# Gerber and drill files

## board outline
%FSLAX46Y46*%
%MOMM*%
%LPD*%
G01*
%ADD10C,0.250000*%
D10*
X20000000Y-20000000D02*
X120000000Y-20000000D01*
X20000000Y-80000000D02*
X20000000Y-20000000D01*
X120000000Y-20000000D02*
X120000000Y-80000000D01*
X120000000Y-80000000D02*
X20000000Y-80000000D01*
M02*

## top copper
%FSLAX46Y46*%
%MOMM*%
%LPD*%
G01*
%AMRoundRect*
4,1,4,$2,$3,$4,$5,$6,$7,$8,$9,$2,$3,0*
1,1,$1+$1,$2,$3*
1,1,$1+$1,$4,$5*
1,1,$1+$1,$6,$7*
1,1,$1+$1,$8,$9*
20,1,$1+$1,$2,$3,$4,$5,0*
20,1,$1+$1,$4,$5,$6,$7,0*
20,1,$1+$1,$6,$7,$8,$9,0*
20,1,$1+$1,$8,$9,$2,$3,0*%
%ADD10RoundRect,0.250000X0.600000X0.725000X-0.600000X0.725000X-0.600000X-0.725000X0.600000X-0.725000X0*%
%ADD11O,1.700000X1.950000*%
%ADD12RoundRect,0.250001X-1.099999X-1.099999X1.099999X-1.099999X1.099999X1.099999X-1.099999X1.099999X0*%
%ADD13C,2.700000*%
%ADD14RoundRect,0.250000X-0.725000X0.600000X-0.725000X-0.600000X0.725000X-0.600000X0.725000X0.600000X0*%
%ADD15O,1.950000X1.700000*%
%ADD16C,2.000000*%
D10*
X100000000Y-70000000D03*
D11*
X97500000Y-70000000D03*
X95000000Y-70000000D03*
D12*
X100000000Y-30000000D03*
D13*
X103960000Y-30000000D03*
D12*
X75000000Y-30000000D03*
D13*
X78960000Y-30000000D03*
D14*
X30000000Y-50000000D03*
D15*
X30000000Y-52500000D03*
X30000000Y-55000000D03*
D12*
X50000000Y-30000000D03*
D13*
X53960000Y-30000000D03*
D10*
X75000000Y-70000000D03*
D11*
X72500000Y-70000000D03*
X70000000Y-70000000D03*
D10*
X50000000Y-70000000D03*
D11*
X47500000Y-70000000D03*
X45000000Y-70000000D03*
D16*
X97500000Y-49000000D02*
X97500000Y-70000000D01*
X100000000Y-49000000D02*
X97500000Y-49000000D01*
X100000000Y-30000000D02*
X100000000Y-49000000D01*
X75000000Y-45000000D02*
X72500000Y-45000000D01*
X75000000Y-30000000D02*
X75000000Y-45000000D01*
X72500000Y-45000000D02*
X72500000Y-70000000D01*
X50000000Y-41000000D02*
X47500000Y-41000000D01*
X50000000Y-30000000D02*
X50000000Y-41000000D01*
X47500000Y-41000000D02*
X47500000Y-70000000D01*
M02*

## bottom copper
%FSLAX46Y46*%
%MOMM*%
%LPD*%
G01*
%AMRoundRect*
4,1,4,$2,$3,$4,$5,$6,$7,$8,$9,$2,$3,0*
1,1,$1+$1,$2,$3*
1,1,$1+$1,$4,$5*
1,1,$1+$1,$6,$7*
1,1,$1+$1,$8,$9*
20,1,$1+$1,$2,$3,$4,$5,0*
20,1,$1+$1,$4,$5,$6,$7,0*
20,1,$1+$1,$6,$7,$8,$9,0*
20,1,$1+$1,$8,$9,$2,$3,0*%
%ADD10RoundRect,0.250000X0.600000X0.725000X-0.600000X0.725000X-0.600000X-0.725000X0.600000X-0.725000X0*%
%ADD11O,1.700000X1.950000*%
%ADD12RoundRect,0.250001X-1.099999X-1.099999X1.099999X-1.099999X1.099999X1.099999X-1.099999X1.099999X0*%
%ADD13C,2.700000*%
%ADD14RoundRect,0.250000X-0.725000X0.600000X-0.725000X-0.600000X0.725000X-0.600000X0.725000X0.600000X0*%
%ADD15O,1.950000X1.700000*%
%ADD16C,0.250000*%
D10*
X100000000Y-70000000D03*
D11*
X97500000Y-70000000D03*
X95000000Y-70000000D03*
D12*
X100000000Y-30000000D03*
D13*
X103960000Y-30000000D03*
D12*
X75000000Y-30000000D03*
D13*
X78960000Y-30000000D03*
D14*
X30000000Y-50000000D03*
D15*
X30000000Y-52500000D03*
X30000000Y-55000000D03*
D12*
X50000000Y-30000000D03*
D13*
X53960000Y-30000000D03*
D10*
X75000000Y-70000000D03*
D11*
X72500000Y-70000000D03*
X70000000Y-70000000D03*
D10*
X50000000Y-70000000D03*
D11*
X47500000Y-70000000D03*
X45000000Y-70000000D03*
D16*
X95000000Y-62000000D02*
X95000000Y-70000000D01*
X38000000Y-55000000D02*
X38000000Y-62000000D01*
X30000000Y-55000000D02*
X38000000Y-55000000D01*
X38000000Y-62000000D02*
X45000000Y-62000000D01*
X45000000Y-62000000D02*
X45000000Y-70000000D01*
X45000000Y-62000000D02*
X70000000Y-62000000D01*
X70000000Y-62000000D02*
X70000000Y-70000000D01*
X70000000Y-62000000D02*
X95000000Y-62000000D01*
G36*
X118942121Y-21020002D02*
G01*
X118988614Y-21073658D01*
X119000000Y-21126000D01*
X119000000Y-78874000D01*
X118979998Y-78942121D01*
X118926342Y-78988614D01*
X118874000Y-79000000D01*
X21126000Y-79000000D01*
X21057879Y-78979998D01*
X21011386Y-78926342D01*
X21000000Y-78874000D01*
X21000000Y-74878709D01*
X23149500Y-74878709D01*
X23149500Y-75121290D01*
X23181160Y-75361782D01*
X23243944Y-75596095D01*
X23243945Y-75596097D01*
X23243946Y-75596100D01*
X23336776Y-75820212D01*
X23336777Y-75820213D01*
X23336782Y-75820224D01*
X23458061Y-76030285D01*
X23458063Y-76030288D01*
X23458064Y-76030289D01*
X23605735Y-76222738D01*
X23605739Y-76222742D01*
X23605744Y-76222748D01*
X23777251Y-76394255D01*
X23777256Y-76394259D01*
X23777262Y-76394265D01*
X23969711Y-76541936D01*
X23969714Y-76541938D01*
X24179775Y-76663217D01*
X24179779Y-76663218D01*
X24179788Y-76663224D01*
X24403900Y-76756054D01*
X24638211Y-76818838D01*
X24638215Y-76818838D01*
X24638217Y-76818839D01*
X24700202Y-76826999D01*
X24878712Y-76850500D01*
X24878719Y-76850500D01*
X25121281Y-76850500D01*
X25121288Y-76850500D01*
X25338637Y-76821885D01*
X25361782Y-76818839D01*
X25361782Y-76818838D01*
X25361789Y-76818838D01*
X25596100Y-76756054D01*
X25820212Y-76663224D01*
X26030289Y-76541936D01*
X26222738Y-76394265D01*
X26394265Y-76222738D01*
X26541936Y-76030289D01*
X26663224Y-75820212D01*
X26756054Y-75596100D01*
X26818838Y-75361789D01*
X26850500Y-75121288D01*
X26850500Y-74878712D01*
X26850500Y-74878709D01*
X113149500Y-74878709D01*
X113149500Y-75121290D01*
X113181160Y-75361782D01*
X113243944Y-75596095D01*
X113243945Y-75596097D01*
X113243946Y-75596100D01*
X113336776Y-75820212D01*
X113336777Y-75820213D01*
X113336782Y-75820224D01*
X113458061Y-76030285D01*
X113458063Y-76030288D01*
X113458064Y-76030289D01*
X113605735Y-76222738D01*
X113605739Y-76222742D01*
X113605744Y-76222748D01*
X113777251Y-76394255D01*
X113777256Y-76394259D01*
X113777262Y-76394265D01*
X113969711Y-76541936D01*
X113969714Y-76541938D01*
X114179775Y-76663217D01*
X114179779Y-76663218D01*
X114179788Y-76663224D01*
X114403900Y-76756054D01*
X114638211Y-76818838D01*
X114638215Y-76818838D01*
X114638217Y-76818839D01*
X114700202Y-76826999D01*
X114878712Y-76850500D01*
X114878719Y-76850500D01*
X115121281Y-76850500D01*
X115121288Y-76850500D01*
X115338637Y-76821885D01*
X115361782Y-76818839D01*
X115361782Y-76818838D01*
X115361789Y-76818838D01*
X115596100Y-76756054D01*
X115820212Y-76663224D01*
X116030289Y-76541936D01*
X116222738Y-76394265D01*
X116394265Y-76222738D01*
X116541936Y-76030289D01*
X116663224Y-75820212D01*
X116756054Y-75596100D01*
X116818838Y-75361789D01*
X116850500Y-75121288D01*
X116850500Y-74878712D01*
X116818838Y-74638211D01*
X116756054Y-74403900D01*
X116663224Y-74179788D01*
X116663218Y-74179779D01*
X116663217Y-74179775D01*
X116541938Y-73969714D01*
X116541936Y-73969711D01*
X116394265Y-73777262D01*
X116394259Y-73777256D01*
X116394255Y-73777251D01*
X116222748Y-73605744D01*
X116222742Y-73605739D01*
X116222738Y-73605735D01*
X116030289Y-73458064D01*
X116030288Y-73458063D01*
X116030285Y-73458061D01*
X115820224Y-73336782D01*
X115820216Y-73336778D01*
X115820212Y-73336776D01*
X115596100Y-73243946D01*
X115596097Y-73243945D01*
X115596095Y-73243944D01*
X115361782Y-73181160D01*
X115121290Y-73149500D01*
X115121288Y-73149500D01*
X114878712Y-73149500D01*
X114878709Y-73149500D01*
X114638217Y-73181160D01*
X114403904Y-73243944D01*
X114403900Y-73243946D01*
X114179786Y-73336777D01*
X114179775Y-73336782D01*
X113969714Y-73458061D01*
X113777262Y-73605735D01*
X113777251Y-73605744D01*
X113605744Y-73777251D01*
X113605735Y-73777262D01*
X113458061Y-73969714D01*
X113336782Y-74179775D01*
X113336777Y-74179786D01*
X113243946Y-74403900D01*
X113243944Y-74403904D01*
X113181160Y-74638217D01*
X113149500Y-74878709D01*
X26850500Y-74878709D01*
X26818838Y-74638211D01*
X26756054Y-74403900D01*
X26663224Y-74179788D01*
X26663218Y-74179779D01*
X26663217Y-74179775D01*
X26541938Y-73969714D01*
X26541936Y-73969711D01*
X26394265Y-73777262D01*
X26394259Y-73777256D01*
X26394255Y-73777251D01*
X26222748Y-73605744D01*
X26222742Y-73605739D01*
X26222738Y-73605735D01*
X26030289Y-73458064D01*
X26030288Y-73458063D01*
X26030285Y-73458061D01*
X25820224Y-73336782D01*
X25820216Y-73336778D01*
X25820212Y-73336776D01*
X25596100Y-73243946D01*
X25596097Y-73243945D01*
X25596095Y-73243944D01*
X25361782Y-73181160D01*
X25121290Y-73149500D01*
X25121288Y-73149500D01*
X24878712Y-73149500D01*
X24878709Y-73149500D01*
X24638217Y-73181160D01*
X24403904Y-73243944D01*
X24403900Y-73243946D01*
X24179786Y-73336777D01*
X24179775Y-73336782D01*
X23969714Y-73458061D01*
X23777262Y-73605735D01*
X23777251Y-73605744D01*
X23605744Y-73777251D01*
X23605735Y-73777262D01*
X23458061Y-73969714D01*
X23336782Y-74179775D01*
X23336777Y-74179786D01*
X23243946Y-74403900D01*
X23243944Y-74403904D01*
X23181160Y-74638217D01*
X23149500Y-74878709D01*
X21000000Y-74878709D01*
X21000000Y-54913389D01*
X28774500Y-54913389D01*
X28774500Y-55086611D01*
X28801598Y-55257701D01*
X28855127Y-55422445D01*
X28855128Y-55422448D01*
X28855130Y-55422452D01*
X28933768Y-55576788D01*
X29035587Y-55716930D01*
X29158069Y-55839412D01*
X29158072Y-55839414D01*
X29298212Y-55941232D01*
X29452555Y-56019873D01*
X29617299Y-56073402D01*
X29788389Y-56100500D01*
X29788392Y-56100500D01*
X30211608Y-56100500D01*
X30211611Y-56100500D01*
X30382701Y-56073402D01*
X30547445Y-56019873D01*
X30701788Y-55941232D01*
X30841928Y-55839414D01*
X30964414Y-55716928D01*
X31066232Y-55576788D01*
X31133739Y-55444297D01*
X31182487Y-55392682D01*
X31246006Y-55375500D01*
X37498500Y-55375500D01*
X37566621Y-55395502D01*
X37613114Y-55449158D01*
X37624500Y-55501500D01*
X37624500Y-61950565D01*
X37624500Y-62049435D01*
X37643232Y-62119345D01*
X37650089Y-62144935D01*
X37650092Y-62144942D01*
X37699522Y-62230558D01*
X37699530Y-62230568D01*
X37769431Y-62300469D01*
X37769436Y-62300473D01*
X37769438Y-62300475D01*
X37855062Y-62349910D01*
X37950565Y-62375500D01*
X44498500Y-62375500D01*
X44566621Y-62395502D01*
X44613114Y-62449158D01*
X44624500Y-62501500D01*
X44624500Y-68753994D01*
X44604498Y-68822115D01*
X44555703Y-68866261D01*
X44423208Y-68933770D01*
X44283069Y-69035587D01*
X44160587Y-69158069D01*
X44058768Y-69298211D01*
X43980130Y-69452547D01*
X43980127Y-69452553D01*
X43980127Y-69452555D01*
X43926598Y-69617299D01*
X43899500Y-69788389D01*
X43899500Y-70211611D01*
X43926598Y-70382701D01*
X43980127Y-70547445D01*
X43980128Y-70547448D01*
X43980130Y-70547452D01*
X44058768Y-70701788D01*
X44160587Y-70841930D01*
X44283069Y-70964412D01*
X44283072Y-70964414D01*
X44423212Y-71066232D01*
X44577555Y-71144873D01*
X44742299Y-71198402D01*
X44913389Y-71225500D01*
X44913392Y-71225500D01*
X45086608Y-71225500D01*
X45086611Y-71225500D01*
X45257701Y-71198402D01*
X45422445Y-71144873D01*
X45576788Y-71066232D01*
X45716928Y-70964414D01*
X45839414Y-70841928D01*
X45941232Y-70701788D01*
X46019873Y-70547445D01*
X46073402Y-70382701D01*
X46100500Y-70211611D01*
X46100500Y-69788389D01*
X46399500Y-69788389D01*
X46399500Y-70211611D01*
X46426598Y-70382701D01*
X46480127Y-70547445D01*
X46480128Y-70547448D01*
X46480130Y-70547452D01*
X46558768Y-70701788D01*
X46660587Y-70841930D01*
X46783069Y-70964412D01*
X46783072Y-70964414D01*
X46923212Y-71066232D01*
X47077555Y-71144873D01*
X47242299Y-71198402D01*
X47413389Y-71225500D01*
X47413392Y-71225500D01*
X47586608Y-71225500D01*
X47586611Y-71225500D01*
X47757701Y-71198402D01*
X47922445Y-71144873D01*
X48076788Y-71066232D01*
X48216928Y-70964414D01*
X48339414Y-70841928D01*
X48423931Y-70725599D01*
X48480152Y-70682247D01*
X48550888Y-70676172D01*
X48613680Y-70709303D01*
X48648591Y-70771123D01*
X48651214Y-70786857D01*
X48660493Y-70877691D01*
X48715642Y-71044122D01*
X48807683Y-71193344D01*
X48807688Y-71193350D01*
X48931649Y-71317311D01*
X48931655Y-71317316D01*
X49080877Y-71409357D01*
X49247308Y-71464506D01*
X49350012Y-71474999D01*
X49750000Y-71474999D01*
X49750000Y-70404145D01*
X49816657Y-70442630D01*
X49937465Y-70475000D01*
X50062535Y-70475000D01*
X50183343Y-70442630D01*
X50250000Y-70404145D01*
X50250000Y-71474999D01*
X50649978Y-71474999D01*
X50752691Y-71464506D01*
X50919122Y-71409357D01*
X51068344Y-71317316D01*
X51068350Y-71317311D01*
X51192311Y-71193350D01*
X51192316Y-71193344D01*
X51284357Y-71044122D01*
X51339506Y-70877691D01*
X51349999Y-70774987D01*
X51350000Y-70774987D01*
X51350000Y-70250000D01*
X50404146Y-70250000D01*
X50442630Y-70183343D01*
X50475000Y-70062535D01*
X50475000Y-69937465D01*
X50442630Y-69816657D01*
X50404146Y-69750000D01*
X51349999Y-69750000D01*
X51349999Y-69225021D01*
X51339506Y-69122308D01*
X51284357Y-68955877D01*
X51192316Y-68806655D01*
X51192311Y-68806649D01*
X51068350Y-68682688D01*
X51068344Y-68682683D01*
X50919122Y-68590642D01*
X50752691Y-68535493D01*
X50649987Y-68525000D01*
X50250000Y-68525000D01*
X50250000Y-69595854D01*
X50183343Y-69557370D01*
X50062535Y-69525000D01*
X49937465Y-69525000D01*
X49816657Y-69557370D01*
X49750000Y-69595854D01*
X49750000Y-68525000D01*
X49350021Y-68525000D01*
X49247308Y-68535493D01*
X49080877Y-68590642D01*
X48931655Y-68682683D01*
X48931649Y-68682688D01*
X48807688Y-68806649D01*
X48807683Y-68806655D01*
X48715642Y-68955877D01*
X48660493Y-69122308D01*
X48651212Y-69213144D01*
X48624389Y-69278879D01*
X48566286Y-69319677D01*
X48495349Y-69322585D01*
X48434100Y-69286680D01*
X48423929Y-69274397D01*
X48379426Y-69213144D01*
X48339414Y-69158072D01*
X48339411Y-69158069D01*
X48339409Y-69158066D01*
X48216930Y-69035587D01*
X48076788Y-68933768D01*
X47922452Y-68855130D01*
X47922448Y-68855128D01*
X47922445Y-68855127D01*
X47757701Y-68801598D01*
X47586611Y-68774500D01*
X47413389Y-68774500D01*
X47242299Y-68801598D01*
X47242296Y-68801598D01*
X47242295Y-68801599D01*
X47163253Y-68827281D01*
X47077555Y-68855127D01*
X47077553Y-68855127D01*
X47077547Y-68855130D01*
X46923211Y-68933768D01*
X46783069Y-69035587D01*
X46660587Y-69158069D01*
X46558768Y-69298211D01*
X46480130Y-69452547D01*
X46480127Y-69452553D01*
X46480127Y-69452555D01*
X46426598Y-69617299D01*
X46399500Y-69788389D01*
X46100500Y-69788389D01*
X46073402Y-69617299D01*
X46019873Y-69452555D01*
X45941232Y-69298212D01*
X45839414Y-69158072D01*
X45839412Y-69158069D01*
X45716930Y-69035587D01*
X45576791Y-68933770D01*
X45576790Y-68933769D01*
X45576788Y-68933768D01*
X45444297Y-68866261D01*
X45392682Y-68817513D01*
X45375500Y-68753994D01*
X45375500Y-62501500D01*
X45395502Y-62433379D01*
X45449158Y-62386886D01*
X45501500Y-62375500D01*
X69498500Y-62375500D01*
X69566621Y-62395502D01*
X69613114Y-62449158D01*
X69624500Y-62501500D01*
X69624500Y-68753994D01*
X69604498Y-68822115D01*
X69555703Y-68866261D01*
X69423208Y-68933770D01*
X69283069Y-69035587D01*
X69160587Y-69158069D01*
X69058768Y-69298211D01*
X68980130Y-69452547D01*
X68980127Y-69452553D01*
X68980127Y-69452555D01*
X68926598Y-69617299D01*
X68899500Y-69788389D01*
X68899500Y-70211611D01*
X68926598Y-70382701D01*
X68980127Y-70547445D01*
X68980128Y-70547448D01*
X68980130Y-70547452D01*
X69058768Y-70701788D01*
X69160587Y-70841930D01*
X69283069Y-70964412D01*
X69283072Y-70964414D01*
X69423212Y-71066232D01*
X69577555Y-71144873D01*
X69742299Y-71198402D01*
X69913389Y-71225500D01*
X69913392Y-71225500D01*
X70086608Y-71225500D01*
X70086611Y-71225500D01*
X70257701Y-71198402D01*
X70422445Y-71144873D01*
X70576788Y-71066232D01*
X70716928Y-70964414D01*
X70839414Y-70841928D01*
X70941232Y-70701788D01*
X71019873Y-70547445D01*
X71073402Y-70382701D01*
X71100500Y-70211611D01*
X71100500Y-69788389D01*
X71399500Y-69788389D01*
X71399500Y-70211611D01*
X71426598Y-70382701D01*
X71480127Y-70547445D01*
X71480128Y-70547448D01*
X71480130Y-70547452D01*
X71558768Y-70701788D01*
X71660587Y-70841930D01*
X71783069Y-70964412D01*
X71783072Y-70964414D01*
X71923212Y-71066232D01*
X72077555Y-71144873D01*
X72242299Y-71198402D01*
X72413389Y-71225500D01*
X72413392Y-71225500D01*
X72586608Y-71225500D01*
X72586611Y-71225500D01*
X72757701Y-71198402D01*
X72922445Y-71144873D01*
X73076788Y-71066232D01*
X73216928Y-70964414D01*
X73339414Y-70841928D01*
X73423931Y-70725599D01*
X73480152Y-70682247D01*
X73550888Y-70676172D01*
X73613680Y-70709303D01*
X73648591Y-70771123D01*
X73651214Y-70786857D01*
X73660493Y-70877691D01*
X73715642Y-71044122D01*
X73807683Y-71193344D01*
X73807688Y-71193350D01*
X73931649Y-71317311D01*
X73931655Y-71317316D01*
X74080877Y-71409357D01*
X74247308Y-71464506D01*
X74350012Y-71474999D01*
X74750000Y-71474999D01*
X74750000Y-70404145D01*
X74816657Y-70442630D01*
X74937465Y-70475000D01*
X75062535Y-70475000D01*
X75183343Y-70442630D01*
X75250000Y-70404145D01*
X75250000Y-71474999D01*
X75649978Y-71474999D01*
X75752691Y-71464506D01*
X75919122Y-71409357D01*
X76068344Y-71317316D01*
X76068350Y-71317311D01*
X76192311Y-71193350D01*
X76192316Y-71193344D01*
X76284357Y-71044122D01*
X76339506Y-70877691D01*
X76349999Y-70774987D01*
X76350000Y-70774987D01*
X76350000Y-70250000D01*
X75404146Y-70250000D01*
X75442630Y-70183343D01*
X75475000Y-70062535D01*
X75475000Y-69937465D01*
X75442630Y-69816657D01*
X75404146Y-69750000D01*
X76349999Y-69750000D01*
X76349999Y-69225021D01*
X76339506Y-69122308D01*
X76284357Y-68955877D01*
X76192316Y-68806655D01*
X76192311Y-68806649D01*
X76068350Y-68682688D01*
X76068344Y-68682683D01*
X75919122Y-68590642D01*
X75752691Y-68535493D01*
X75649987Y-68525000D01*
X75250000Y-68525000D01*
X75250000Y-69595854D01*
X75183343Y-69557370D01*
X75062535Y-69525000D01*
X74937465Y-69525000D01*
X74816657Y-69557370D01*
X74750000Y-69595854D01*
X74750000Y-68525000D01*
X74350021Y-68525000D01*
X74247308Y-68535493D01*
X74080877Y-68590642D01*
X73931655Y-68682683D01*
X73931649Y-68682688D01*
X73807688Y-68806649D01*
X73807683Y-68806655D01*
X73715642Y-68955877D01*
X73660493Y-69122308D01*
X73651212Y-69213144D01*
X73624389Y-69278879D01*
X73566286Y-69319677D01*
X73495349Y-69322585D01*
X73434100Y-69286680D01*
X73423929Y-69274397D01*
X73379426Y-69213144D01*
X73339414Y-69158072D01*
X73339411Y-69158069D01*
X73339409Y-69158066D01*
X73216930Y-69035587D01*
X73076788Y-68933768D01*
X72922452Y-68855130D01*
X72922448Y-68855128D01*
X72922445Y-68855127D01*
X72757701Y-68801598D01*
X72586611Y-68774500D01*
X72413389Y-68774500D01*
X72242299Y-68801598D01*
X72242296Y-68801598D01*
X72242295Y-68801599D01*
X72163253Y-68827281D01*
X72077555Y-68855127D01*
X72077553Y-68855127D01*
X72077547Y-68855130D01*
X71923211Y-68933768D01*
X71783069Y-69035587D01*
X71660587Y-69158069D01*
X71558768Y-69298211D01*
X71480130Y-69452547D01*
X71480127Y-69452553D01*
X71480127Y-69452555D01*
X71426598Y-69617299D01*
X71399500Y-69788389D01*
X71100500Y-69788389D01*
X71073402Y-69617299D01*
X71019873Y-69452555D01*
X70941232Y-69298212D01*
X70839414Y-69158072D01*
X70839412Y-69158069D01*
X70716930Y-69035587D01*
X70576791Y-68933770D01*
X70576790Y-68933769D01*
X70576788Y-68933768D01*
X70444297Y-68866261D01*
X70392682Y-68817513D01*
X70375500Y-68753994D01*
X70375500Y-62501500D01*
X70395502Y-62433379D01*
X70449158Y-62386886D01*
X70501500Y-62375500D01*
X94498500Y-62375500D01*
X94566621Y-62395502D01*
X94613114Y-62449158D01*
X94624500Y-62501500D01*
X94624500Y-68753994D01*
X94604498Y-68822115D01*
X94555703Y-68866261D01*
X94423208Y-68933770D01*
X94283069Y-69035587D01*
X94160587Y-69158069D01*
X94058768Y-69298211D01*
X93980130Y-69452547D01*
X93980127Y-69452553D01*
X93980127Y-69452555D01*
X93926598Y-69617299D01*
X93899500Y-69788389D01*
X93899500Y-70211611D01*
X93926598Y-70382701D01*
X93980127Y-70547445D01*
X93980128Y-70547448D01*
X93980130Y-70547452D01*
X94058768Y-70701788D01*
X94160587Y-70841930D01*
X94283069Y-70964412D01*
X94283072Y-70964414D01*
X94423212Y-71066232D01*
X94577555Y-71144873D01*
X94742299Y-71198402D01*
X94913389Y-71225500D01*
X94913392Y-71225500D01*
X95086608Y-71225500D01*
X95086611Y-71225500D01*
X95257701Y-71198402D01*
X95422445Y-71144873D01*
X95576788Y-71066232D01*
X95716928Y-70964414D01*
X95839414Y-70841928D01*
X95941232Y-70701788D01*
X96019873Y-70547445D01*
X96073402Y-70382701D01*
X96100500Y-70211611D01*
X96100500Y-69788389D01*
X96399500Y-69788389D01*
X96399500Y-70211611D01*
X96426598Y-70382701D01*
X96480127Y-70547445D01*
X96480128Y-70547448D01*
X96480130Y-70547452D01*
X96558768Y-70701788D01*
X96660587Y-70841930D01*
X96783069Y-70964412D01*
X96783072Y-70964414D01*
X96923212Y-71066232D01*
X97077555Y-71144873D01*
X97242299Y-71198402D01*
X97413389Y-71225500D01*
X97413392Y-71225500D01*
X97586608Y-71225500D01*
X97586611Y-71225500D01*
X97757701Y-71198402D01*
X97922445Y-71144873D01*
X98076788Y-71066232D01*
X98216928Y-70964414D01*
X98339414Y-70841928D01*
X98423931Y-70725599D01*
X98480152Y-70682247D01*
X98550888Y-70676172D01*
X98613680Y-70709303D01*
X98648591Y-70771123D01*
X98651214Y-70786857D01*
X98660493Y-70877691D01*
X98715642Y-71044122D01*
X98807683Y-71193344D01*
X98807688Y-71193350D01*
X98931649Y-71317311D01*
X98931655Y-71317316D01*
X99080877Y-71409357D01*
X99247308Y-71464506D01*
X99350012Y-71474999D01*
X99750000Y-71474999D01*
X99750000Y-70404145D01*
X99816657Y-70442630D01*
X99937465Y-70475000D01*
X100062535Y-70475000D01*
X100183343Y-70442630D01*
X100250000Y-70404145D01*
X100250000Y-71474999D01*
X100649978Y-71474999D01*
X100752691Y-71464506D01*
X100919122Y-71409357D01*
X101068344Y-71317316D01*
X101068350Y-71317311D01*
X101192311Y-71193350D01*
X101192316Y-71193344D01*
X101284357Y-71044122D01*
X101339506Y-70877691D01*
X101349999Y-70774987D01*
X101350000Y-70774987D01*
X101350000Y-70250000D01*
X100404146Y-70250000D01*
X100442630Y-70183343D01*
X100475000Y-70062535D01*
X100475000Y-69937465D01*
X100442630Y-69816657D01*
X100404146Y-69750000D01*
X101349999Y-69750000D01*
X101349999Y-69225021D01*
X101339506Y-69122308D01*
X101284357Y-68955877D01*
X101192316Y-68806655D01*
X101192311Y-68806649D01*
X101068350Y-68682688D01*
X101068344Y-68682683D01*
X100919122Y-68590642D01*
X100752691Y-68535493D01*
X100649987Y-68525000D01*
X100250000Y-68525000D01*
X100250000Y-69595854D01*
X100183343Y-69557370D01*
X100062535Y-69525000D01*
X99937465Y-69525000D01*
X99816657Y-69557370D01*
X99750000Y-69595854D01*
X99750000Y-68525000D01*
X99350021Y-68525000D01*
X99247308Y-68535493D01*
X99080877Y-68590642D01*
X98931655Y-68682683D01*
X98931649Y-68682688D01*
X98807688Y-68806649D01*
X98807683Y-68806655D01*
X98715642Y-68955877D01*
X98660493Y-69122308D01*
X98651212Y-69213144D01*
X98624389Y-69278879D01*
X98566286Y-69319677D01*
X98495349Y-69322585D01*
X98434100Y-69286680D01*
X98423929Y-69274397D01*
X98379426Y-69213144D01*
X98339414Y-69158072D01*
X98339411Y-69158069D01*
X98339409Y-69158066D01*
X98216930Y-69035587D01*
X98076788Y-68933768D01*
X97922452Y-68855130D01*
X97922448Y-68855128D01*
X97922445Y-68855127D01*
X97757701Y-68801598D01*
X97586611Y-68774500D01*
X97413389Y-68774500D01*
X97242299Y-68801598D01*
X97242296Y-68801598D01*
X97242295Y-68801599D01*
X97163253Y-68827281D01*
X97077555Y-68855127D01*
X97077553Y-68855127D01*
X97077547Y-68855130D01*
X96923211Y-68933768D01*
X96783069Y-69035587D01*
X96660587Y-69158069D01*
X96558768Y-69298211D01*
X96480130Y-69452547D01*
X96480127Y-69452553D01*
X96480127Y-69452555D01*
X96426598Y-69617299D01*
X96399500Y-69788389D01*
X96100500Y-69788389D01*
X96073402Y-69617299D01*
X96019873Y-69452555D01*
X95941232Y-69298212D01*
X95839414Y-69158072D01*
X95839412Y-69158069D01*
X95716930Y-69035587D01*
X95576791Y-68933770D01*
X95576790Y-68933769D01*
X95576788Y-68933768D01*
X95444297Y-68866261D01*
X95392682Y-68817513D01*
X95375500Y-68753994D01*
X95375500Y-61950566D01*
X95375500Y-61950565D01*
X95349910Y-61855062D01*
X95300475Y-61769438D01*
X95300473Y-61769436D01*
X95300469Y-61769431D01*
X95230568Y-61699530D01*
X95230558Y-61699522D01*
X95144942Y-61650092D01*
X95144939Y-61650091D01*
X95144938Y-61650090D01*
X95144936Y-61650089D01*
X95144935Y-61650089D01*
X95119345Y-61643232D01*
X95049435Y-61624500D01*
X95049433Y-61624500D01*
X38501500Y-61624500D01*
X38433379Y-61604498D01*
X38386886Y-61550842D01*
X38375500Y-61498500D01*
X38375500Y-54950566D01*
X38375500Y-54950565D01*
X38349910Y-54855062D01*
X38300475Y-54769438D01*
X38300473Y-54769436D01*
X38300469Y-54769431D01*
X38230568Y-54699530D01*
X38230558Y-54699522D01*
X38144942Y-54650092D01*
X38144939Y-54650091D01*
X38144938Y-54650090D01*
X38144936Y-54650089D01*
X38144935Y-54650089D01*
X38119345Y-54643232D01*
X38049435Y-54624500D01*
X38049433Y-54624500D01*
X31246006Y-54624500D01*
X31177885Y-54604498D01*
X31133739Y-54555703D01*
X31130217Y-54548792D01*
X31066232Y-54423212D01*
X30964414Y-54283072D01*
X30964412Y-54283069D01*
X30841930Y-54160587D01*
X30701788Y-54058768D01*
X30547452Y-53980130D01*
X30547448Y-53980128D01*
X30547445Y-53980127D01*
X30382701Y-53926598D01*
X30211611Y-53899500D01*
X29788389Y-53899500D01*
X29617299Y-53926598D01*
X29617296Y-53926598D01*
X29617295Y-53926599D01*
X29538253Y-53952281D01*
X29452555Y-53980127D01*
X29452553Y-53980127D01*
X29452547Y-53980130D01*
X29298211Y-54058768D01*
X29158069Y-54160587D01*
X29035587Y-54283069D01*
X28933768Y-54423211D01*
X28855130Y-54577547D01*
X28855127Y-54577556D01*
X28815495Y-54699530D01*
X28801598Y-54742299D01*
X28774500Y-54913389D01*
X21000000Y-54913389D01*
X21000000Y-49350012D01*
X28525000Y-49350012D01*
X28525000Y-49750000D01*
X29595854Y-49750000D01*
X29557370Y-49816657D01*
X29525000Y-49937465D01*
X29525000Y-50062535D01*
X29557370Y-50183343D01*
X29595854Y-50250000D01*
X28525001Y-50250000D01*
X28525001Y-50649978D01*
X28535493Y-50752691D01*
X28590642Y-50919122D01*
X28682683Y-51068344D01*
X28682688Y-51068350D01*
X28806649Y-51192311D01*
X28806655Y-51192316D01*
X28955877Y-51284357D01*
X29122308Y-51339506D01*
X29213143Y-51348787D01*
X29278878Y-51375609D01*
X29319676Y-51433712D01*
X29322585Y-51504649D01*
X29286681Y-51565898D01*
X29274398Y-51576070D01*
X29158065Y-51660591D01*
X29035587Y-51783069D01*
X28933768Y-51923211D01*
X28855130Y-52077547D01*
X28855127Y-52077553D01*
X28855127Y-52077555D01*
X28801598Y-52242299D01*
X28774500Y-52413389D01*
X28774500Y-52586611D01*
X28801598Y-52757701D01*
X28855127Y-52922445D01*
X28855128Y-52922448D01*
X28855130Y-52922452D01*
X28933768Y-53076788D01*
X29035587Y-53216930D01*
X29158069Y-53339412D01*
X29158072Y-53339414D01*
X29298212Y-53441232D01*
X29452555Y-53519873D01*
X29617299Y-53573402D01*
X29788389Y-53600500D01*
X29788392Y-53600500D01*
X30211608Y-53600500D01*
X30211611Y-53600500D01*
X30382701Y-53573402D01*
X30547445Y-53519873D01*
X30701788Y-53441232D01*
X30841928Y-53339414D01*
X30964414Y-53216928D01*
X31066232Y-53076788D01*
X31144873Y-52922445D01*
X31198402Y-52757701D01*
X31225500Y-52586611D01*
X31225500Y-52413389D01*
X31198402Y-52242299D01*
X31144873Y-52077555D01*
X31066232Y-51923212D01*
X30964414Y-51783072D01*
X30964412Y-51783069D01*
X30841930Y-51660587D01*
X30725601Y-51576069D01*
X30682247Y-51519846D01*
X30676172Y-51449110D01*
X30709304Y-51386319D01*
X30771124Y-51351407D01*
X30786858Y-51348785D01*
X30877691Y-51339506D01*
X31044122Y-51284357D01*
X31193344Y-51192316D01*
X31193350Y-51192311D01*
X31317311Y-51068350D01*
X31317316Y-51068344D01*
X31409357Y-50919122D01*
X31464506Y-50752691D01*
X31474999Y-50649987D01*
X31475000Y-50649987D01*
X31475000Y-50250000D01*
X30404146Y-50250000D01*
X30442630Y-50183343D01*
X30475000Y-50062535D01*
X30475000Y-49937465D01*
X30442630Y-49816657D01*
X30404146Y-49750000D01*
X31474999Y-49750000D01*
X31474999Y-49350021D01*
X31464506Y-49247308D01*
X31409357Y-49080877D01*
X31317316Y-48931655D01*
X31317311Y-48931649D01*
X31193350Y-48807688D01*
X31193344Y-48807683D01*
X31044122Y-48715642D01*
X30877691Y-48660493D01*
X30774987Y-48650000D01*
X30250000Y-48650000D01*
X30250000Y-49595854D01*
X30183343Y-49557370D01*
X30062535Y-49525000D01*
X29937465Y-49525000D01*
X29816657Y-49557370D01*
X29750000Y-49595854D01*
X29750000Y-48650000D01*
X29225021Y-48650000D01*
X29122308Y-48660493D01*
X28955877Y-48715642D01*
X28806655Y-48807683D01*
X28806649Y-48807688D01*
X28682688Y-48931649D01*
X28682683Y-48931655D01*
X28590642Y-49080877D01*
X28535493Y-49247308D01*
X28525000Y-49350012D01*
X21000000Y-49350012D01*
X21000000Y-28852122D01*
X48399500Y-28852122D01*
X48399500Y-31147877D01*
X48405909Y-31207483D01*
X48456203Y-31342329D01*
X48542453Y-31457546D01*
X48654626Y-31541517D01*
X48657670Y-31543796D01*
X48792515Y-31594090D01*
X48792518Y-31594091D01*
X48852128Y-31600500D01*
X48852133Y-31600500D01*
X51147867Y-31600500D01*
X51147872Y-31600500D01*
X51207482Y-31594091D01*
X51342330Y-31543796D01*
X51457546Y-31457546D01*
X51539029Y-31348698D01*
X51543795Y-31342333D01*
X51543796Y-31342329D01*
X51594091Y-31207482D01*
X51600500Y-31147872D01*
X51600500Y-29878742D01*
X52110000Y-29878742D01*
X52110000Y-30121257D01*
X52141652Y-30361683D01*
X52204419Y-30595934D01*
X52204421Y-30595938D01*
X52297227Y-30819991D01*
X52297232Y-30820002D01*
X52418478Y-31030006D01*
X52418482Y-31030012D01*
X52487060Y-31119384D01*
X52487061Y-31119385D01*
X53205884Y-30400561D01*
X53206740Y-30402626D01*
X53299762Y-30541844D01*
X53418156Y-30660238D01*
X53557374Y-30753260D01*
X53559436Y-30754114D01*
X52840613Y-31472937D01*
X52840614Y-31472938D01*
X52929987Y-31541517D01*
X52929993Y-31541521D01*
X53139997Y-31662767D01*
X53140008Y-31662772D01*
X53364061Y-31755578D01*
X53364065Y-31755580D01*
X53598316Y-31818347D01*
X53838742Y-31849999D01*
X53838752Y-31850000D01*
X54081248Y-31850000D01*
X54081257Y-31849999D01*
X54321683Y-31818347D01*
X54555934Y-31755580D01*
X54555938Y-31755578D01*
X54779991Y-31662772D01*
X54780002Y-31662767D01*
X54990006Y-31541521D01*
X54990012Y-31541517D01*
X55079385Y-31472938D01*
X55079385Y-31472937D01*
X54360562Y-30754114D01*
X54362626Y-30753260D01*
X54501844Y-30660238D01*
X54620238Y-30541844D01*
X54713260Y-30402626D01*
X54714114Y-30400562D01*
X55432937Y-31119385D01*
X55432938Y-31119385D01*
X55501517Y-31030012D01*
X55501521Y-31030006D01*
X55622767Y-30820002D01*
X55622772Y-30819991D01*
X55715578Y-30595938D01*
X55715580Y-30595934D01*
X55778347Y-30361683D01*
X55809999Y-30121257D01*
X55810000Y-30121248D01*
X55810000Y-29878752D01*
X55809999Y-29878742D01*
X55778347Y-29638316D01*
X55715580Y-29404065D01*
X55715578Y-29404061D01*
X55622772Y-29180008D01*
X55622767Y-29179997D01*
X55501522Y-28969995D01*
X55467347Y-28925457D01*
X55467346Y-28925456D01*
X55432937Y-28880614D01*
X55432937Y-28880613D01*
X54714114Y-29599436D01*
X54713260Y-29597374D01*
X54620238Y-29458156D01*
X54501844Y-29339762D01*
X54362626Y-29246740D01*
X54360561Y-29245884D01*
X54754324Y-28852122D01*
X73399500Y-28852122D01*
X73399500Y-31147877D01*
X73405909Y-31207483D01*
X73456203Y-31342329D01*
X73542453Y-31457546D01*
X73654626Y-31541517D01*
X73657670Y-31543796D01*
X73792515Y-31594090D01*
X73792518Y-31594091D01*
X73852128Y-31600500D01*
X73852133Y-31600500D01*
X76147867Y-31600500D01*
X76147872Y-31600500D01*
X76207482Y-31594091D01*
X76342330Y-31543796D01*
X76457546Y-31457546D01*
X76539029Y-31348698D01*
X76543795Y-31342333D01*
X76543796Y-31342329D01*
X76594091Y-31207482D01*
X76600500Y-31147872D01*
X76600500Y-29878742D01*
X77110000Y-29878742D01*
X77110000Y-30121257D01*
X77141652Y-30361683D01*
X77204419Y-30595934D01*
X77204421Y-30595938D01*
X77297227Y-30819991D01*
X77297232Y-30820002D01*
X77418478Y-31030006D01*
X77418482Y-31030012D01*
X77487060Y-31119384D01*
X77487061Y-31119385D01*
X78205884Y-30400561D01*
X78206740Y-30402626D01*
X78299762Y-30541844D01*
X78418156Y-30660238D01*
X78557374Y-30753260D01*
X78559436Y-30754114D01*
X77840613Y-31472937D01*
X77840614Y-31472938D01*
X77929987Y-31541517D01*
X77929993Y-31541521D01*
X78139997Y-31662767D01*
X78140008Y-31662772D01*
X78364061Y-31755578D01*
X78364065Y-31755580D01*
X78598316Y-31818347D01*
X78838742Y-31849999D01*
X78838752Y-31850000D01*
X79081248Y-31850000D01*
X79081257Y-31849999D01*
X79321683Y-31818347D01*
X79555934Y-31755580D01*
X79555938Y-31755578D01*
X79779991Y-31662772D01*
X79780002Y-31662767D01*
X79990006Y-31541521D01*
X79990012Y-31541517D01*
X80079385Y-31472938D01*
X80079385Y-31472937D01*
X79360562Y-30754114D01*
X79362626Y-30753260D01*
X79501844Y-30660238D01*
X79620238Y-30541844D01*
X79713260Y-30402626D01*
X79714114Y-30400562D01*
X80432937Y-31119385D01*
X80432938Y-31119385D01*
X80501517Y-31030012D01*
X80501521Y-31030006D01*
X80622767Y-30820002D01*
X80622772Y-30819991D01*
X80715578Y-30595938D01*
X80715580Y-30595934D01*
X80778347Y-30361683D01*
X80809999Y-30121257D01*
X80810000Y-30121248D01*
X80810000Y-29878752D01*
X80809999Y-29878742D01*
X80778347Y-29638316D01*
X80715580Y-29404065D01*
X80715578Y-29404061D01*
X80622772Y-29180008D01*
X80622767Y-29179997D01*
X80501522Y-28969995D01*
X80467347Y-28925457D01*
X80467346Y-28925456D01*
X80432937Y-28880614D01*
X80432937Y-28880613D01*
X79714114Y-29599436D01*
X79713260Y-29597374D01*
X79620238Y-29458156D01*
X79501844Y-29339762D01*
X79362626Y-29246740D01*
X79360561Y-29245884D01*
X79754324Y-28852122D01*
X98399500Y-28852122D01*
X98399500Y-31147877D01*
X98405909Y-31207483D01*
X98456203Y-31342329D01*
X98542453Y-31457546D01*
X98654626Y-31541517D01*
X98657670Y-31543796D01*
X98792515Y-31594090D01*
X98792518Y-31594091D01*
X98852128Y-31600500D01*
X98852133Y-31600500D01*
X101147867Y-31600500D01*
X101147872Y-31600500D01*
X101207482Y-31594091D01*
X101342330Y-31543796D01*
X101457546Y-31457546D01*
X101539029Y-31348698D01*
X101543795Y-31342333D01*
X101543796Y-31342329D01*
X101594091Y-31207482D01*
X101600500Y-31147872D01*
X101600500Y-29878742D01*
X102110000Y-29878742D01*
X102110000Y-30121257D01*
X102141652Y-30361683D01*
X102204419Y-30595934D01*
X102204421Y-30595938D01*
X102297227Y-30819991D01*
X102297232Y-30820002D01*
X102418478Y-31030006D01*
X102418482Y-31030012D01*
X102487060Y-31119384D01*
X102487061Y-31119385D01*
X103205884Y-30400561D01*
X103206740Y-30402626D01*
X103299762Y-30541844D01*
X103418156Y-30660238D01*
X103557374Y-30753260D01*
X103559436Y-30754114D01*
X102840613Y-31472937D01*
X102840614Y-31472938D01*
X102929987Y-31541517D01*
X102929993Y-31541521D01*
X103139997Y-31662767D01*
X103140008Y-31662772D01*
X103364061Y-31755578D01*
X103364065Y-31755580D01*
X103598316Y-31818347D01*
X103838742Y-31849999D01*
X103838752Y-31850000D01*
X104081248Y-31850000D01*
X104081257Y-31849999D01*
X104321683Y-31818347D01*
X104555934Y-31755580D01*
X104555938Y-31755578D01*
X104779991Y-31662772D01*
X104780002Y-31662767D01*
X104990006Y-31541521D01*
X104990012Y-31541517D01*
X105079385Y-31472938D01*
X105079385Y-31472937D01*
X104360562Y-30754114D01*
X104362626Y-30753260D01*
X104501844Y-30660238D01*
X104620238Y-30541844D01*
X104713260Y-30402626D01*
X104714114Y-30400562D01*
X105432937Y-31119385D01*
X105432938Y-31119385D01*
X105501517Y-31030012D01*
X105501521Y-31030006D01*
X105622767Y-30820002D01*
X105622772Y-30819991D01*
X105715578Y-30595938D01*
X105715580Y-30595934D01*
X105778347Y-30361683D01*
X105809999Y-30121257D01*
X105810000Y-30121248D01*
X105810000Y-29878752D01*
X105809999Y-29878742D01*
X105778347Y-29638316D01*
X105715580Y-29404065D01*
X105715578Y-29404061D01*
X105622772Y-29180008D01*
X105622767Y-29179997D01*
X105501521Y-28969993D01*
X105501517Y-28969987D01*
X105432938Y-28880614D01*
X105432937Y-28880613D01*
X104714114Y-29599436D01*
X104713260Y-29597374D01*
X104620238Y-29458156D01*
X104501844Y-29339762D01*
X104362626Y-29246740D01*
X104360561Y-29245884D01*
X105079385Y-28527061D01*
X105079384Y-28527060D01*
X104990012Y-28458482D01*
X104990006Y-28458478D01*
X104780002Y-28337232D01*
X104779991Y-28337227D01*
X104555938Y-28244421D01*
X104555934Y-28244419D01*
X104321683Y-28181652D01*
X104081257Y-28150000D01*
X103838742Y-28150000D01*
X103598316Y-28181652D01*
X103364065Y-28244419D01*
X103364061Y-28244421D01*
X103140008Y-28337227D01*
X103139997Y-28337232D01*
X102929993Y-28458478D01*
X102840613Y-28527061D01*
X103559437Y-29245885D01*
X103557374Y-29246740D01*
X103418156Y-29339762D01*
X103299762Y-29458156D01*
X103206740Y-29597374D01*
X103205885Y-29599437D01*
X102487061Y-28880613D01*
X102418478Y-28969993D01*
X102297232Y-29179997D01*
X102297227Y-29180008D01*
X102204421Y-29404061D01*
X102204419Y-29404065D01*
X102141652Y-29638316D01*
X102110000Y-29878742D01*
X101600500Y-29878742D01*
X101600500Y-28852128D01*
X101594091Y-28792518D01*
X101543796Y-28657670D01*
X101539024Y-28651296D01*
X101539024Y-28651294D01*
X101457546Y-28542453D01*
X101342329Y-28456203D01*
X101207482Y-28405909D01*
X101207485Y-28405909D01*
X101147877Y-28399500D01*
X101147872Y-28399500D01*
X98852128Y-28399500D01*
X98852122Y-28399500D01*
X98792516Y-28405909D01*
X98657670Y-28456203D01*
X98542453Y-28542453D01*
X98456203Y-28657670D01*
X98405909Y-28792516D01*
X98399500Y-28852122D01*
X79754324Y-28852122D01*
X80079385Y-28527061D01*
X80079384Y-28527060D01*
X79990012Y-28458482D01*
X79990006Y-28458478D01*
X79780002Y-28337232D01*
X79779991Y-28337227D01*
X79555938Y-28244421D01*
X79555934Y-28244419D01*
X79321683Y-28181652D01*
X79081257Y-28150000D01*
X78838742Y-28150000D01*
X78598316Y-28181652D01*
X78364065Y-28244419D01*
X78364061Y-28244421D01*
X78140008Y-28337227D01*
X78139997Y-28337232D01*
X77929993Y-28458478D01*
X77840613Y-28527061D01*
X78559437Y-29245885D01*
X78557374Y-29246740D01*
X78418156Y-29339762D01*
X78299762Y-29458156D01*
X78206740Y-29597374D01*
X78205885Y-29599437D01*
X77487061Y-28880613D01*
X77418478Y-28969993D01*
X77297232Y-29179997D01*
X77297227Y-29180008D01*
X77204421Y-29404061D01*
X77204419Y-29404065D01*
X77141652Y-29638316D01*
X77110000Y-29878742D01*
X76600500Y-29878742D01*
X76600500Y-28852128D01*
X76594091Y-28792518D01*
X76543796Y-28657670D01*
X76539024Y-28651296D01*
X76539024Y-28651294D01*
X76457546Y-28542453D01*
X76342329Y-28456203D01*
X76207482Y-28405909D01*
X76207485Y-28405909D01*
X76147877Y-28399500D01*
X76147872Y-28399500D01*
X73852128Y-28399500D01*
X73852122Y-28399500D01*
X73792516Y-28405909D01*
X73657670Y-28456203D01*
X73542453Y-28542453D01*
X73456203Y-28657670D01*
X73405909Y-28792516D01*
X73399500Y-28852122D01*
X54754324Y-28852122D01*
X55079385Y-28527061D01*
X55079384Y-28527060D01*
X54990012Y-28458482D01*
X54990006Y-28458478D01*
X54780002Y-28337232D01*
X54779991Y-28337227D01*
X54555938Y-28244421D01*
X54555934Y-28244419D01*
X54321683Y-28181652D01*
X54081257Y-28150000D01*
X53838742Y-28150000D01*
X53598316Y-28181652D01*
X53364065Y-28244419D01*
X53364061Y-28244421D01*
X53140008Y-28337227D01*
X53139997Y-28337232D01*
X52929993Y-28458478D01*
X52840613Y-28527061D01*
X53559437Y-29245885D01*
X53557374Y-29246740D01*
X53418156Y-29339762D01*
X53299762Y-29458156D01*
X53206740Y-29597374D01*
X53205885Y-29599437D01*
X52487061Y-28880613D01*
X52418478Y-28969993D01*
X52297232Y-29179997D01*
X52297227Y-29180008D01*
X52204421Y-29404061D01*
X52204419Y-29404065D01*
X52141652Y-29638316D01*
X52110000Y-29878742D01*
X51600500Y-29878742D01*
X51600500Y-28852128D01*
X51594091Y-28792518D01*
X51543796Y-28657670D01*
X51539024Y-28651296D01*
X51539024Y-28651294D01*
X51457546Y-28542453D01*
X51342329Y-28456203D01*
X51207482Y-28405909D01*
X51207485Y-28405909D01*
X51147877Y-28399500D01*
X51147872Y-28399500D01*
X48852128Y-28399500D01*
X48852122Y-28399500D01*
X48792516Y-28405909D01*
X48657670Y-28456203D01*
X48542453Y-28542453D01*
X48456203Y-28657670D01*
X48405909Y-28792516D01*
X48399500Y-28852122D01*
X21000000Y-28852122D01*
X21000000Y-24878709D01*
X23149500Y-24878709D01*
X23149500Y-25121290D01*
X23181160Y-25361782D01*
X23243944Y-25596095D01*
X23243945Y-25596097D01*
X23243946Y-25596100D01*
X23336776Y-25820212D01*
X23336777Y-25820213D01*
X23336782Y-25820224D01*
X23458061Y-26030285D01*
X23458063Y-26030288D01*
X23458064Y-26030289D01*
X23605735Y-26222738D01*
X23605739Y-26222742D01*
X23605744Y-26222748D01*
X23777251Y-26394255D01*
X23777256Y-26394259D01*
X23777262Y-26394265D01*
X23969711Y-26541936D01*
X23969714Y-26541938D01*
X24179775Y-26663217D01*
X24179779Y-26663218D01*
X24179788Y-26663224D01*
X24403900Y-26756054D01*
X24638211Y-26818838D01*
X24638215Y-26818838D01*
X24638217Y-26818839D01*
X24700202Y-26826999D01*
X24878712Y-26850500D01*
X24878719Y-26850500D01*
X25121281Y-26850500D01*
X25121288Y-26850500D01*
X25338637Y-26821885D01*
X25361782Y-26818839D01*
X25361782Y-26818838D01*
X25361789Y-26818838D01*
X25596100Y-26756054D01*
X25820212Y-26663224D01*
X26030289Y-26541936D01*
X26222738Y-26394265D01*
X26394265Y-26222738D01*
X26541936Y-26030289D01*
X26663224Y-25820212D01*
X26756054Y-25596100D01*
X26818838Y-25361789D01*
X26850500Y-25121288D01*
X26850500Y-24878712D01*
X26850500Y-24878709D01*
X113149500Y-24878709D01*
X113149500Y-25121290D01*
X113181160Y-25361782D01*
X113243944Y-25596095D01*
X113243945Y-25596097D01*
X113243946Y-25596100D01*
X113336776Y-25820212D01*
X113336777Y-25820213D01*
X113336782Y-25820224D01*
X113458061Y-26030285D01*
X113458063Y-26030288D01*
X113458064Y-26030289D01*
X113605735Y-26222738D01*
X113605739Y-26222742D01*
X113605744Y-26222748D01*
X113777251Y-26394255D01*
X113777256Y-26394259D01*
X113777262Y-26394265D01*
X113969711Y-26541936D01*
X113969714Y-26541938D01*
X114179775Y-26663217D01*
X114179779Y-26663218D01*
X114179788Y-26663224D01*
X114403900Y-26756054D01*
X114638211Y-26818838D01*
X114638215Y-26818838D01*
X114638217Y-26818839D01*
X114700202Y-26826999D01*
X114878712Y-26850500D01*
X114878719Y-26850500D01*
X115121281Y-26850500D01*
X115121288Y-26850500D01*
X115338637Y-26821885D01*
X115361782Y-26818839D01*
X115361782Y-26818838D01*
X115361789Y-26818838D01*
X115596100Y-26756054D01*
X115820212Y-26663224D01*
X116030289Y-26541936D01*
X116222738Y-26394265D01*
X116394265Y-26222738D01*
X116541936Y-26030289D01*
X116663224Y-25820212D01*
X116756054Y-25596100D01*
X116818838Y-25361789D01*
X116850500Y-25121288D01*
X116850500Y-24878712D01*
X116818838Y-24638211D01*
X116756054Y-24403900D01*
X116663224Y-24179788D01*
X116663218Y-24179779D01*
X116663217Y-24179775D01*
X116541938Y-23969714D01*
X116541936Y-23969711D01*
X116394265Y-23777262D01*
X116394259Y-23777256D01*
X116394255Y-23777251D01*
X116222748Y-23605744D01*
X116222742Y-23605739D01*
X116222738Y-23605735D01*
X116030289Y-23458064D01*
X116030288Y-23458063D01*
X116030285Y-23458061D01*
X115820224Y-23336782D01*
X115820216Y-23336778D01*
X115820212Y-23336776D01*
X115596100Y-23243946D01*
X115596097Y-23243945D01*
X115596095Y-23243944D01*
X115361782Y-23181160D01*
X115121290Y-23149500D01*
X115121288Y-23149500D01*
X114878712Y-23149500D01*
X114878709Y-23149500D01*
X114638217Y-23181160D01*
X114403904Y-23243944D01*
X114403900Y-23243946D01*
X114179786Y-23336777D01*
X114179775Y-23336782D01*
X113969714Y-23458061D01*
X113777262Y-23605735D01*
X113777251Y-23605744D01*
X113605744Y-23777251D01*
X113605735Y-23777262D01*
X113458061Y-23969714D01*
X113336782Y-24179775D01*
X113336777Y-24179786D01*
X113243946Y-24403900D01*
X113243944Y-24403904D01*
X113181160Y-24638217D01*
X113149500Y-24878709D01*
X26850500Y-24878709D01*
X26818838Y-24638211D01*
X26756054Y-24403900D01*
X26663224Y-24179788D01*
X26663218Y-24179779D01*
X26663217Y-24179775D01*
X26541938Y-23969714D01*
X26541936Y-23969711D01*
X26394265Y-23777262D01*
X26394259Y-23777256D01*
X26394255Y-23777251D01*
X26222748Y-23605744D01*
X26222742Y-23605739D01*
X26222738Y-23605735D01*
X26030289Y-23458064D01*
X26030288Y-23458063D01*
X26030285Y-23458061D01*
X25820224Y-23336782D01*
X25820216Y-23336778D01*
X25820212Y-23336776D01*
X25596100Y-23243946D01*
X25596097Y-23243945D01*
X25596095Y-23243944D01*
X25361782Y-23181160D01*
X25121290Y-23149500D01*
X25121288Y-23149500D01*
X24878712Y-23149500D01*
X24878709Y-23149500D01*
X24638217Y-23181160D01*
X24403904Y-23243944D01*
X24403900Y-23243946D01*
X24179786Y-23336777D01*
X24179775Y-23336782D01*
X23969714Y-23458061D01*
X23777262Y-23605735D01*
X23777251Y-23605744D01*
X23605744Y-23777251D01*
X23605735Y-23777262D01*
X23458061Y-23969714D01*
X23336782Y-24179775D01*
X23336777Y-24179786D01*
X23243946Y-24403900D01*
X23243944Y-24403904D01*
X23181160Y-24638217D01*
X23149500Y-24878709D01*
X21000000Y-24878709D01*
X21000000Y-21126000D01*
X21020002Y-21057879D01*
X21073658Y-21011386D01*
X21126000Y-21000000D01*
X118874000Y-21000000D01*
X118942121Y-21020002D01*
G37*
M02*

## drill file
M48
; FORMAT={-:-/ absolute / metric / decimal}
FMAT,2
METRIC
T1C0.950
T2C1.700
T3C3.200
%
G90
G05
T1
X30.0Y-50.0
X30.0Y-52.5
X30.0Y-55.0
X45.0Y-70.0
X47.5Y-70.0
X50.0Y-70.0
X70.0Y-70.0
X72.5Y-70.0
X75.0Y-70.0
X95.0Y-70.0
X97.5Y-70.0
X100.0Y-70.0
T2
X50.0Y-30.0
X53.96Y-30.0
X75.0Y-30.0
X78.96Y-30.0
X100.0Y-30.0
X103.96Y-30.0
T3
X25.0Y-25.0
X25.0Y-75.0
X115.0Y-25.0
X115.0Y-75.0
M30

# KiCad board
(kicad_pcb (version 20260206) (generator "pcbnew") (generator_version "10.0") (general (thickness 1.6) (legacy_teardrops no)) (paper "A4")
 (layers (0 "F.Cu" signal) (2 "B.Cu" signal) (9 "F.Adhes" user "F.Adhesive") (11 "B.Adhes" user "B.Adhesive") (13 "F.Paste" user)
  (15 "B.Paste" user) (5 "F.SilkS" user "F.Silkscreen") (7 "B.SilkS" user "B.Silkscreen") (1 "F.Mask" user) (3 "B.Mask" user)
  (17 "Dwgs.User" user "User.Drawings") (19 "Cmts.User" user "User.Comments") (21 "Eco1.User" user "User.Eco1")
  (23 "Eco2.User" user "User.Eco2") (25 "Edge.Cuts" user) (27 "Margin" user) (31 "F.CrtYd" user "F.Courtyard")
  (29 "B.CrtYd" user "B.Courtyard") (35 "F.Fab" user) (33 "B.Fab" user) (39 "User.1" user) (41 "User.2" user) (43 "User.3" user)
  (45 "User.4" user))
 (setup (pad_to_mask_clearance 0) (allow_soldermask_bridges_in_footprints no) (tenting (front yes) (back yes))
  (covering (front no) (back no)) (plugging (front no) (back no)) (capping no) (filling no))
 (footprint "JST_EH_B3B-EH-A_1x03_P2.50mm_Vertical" (layer "F.Cu") (at 100 70 180)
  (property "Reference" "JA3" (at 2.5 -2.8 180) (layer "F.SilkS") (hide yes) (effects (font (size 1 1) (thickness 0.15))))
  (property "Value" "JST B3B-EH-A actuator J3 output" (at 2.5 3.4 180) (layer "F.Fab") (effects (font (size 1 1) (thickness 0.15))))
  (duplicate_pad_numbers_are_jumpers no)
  (pad "1" thru_hole roundrect (at 0 0 180) (size 1.7 1.95) (drill 0.95) (layers "*.Cu" "*.Mask") (remove_unused_layers no)
   (roundrect_rratio 0.147059) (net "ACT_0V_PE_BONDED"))
  (pad "2" thru_hole oval (at 2.5 0 180) (size 1.7 1.95) (drill 0.95) (layers "*.Cu" "*.Mask") (remove_unused_layers no) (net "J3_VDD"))
  (pad "3" thru_hole oval (at 5 0 180) (size 1.7 1.95) (drill 0.95) (layers "*.Cu" "*.Mask") (remove_unused_layers no) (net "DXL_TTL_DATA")))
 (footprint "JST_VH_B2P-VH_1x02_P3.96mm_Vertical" (layer "F.Cu") (at 100 30)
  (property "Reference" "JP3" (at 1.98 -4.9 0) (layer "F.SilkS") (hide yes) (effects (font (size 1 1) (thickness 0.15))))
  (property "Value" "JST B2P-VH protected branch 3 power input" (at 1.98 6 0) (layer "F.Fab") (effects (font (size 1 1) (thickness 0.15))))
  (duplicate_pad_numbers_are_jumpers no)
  (pad "1" thru_hole roundrect (at 0 0) (size 2.7 2.7) (drill 1.7) (layers "*.Cu" "*.Mask") (remove_unused_layers no)
   (roundrect_rratio 0.092593) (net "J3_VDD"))
  (pad "2" thru_hole circle (at 3.96 0) (size 2.7 2.7) (drill 1.7) (layers "*.Cu" "*.Mask") (remove_unused_layers no)
   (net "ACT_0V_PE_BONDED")))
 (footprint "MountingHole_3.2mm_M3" (layer "F.Cu") (at 115 25)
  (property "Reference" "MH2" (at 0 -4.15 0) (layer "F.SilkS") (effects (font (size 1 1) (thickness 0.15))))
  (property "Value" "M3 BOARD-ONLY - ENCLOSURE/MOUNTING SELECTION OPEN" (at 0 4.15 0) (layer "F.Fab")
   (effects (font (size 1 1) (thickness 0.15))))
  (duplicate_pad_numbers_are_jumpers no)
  (pad "" np_thru_hole circle (at 0 0) (size 3.2 3.2) (drill 3.2) (layers "*.Cu" "*.Mask")))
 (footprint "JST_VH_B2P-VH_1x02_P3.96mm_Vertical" (layer "F.Cu") (at 75 30)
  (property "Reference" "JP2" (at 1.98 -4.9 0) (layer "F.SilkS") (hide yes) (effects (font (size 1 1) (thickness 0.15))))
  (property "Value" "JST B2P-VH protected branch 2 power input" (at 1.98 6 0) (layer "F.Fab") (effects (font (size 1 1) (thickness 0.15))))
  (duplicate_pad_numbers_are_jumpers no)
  (pad "1" thru_hole roundrect (at 0 0) (size 2.7 2.7) (drill 1.7) (layers "*.Cu" "*.Mask") (remove_unused_layers no)
   (roundrect_rratio 0.092593) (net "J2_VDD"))
  (pad "2" thru_hole circle (at 3.96 0) (size 2.7 2.7) (drill 1.7) (layers "*.Cu" "*.Mask") (remove_unused_layers no)
   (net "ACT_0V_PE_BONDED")))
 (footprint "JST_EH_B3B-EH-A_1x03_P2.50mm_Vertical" (layer "F.Cu") (at 30 50 -90)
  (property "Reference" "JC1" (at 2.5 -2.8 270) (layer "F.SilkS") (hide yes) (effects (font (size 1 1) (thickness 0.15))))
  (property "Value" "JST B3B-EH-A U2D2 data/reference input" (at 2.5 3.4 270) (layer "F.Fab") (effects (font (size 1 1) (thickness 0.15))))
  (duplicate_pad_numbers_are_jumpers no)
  (pad "1" thru_hole roundrect (at 0 0 270) (size 1.7 1.95) (drill 0.95) (layers "*.Cu" "*.Mask") (remove_unused_layers no)
   (roundrect_rratio 0.147059) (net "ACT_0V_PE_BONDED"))
  (pad "2" thru_hole oval (at 2.5 0 270) (size 1.7 1.95) (drill 0.95) (layers "*.Cu" "*.Mask") (remove_unused_layers no))
  (pad "3" thru_hole oval (at 5 0 270) (size 1.7 1.95) (drill 0.95) (layers "*.Cu" "*.Mask") (remove_unused_layers no) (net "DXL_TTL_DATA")))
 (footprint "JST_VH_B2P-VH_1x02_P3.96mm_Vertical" (layer "F.Cu") (at 50 30)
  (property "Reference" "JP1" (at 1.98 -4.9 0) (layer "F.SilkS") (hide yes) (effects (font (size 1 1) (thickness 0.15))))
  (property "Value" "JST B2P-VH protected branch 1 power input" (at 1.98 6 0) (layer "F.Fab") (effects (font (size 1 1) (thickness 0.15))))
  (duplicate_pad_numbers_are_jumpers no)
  (pad "1" thru_hole roundrect (at 0 0) (size 2.7 2.7) (drill 1.7) (layers "*.Cu" "*.Mask") (remove_unused_layers no)
   (roundrect_rratio 0.092593) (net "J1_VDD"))
  (pad "2" thru_hole circle (at 3.96 0) (size 2.7 2.7) (drill 1.7) (layers "*.Cu" "*.Mask") (remove_unused_layers no)
   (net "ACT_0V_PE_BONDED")))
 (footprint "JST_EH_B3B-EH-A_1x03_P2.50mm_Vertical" (layer "F.Cu") (at 75 70 180)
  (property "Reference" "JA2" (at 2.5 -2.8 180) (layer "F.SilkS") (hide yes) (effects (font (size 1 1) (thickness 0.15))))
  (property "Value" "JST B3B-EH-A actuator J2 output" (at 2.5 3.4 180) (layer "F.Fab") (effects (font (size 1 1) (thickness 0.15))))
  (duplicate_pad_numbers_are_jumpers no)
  (pad "1" thru_hole roundrect (at 0 0 180) (size 1.7 1.95) (drill 0.95) (layers "*.Cu" "*.Mask") (remove_unused_layers no)
   (roundrect_rratio 0.147059) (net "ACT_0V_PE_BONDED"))
  (pad "2" thru_hole oval (at 2.5 0 180) (size 1.7 1.95) (drill 0.95) (layers "*.Cu" "*.Mask") (remove_unused_layers no) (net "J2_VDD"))
  (pad "3" thru_hole oval (at 5 0 180) (size 1.7 1.95) (drill 0.95) (layers "*.Cu" "*.Mask") (remove_unused_layers no) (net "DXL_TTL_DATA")))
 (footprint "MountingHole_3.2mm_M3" (layer "F.Cu") (at 25 25)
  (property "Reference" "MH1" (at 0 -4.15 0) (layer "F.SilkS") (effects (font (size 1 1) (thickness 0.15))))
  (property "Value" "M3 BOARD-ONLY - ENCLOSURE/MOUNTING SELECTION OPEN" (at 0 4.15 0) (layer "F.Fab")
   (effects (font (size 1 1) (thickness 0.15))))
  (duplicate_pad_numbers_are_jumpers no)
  (pad "" np_thru_hole circle (at 0 0) (size 3.2 3.2) (drill 3.2) (layers "*.Cu" "*.Mask")))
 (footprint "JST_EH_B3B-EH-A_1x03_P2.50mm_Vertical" (layer "F.Cu") (at 50 70 180)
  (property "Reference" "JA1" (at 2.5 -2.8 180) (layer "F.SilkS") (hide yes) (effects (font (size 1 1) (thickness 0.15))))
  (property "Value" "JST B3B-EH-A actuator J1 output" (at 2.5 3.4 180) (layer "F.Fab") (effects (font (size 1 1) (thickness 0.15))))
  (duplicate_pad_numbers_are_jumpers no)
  (pad "1" thru_hole roundrect (at 0 0 180) (size 1.7 1.95) (drill 0.95) (layers "*.Cu" "*.Mask") (remove_unused_layers no)
   (roundrect_rratio 0.147059) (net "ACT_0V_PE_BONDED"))
  (pad "2" thru_hole oval (at 2.5 0 180) (size 1.7 1.95) (drill 0.95) (layers "*.Cu" "*.Mask") (remove_unused_layers no) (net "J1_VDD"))
  (pad "3" thru_hole oval (at 5 0 180) (size 1.7 1.95) (drill 0.95) (layers "*.Cu" "*.Mask") (remove_unused_layers no) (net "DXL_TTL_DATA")))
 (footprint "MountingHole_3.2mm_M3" (layer "F.Cu") (at 115 75)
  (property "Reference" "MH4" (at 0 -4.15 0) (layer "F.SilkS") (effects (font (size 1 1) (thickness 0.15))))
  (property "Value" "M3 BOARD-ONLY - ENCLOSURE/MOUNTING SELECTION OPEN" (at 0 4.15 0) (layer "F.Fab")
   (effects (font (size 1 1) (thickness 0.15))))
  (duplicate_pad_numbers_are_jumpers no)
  (pad "" np_thru_hole circle (at 0 0) (size 3.2 3.2) (drill 3.2) (layers "*.Cu" "*.Mask")))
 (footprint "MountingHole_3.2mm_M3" (layer "F.Cu") (at 25 75)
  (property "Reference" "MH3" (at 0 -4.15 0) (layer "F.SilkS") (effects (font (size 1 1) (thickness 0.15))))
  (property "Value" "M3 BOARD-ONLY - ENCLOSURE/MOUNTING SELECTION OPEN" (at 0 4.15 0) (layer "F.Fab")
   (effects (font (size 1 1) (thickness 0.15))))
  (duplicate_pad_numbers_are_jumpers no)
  (pad "" np_thru_hole circle (at 0 0) (size 3.2 3.2) (drill 3.2) (layers "*.Cu" "*.Mask")))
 (gr_line (start 20 20) (end 120 20) (stroke (width 0.25) (type default)) (layer "Edge.Cuts"))
 (gr_line (start 20 80) (end 20 20) (stroke (width 0.25) (type default)) (layer "Edge.Cuts"))
 (gr_line (start 120 20) (end 120 80) (stroke (width 0.25) (type default)) (layer "Edge.Cuts"))
 (gr_line (start 120 80) (end 20 80) (stroke (width 0.25) (type default)) (layer "Edge.Cuts"))
 (segment (start 97.5 49) (end 97.5 70) (width 2) (layer "F.Cu") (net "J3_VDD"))
 (segment (start 100 49) (end 97.5 49) (width 2) (layer "F.Cu") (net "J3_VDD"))
 (segment (start 100 30) (end 100 49) (width 2) (layer "F.Cu") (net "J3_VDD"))
 (segment (start 95 62) (end 95 70) (width 0.25) (layer "B.Cu") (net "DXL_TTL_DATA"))
 (segment (start 38 55) (end 38 62) (width 0.25) (layer "B.Cu") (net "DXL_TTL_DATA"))
 (segment (start 30 55) (end 38 55) (width 0.25) (layer "B.Cu") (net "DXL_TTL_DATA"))
 (segment (start 38 62) (end 45 62) (width 0.25) (layer "B.Cu") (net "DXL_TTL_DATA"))
 (segment (start 45 62) (end 45 70) (width 0.25) (layer "B.Cu") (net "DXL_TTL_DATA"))
 (segment (start 45 62) (end 70 62) (width 0.25) (layer "B.Cu") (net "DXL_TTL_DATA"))
 (segment (start 70 62) (end 70 70) (width 0.25) (layer "B.Cu") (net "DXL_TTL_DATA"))
 (segment (start 70 62) (end 95 62) (width 0.25) (layer "B.Cu") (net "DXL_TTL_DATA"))
 (segment (start 75 45) (end 72.5 45) (width 2) (layer "F.Cu") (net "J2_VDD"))
 (segment (start 75 30) (end 75 45) (width 2) (layer "F.Cu") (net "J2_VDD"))
 (segment (start 72.5 45) (end 72.5 70) (width 2) (layer "F.Cu") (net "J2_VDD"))
 (segment (start 50 41) (end 47.5 41) (width 2) (layer "F.Cu") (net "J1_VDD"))
 (segment (start 50 30) (end 50 41) (width 2) (layer "F.Cu") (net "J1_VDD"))
 (segment (start 47.5 41) (end 47.5 70) (width 2) (layer "F.Cu") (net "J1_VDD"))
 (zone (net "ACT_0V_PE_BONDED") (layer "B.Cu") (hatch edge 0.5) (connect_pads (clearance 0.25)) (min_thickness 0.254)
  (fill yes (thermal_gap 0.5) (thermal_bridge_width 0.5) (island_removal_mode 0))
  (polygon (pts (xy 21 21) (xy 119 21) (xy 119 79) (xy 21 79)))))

